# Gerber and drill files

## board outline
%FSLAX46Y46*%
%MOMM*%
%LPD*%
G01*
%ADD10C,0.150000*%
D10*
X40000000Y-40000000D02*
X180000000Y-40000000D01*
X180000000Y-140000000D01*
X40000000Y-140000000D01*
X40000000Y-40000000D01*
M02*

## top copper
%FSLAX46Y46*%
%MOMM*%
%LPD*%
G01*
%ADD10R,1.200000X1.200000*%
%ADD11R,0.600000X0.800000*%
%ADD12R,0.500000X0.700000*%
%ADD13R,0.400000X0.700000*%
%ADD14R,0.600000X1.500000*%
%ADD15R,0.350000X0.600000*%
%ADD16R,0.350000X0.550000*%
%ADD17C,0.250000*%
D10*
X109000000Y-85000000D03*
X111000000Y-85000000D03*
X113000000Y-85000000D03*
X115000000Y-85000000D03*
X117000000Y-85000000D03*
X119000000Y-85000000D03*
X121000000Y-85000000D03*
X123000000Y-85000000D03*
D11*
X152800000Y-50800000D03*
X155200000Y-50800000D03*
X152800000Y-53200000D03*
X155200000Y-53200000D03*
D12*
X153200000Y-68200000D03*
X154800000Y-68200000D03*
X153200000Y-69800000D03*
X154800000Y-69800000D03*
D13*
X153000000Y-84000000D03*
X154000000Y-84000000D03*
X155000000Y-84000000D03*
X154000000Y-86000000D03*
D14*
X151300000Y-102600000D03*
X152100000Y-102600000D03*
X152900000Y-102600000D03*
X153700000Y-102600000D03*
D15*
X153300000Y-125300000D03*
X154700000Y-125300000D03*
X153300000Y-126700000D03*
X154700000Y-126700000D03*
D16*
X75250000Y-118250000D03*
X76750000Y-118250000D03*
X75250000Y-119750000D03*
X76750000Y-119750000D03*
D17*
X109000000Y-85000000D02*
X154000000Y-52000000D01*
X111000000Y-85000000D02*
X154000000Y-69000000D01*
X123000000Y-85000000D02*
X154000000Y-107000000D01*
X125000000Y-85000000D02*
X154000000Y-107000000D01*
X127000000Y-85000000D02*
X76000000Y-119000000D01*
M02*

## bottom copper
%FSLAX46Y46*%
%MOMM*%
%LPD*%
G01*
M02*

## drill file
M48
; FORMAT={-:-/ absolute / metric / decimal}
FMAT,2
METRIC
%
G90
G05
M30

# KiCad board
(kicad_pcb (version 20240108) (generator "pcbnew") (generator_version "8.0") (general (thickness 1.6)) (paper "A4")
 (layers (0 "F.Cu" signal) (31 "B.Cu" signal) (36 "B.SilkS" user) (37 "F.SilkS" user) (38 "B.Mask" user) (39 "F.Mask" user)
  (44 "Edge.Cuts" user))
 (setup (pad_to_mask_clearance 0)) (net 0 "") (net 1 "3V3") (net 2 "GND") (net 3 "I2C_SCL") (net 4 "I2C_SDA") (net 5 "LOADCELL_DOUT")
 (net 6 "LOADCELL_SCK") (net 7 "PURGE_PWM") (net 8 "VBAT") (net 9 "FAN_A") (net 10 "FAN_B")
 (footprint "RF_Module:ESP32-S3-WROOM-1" (layer "F.Cu") (at 118 94) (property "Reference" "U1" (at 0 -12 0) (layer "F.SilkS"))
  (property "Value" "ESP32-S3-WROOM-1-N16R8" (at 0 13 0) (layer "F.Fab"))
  (pad "1" smd rect (at -9 -9) (size 1.2 1.2) (layers "F.Cu" "F.Mask") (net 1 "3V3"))
  (pad "2" smd rect (at -7 -9) (size 1.2 1.2) (layers "F.Cu" "F.Mask") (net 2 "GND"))
  (pad "3" smd rect (at -5 -9) (size 1.2 1.2) (layers "F.Cu" "F.Mask") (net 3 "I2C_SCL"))
  (pad "4" smd rect (at -3 -9) (size 1.2 1.2) (layers "F.Cu" "F.Mask") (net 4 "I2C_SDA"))
  (pad "5" smd rect (at -1 -9) (size 1.2 1.2) (layers "F.Cu" "F.Mask") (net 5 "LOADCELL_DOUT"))
  (pad "6" smd rect (at 1 -9) (size 1.2 1.2) (layers "F.Cu" "F.Mask") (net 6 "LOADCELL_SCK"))
  (pad "7" smd rect (at 3 -9) (size 1.2 1.2) (layers "F.Cu" "F.Mask") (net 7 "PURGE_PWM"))
  (pad "8" smd rect (at 5 -9) (size 1.2 1.2) (layers "F.Cu" "F.Mask") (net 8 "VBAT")))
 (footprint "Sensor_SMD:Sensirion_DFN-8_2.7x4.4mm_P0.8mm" (layer "F.Cu") (at 154 52)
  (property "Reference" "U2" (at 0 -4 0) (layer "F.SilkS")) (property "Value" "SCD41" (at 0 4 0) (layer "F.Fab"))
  (pad "1" smd rect (at -1.2 -1.2) (size 0.6 0.8) (layers "F.Cu" "F.Mask") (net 1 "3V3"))
  (pad "2" smd rect (at 1.2 -1.2) (size 0.6 0.8) (layers "F.Cu" "F.Mask") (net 3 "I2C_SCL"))
  (pad "3" smd rect (at -1.2 1.2) (size 0.6 0.8) (layers "F.Cu" "F.Mask") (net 4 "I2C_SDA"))
  (pad "4" smd rect (at 1.2 1.2) (size 0.6 0.8) (layers "F.Cu" "F.Mask") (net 2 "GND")))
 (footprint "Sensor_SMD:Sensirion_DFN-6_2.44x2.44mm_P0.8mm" (layer "F.Cu") (at 154 69)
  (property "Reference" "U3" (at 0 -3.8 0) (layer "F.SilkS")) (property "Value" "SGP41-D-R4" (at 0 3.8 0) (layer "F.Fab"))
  (pad "1" smd rect (at -0.8 -0.8) (size 0.5 0.7) (layers "F.Cu" "F.Mask") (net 1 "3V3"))
  (pad "2" smd rect (at 0.8 -0.8) (size 0.5 0.7) (layers "F.Cu" "F.Mask") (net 3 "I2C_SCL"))
  (pad "3" smd rect (at -0.8 0.8) (size 0.5 0.7) (layers "F.Cu" "F.Mask") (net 4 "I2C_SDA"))
  (pad "4" smd rect (at 0.8 0.8) (size 0.5 0.7) (layers "F.Cu" "F.Mask") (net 2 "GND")))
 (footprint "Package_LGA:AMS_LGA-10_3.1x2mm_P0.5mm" (layer "F.Cu") (at 154 85) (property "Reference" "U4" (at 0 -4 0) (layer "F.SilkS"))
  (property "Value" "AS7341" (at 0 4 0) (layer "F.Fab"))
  (pad "1" smd rect (at -1 -1) (size 0.4 0.7) (layers "F.Cu" "F.Mask") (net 1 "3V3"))
  (pad "2" smd rect (at 0 -1) (size 0.4 0.7) (layers "F.Cu" "F.Mask") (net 3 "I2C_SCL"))
  (pad "3" smd rect (at 1 -1) (size 0.4 0.7) (layers "F.Cu" "F.Mask") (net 4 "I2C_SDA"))
  (pad "4" smd rect (at 0 1) (size 0.4 0.7) (layers "F.Cu" "F.Mask") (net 2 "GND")))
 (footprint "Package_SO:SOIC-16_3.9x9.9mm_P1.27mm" (layer "F.Cu") (at 154 107) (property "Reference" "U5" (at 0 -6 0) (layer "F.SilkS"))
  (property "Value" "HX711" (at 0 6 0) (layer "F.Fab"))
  (pad "1" smd rect (at -2.7 -4.4) (size 0.6 1.5) (layers "F.Cu" "F.Mask") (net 1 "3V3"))
  (pad "2" smd rect (at -1.9 -4.4) (size 0.6 1.5) (layers "F.Cu" "F.Mask") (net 5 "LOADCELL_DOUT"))
  (pad "3" smd rect (at -1.1 -4.4) (size 0.6 1.5) (layers "F.Cu" "F.Mask") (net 6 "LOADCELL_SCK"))
  (pad "4" smd rect (at -0.3 -4.4) (size 0.6 1.5) (layers "F.Cu" "F.Mask") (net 2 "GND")))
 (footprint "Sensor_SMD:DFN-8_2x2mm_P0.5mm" (layer "F.Cu") (at 154 126) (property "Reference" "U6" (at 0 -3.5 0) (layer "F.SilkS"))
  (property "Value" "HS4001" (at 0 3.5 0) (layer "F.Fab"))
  (pad "1" smd rect (at -0.7 -0.7) (size 0.35 0.6) (layers "F.Cu" "F.Mask") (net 1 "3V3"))
  (pad "2" smd rect (at 0.7 -0.7) (size 0.35 0.6) (layers "F.Cu" "F.Mask") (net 3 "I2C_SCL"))
  (pad "3" smd rect (at -0.7 0.7) (size 0.35 0.6) (layers "F.Cu" "F.Mask") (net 4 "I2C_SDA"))
  (pad "4" smd rect (at 0.7 0.7) (size 0.35 0.6) (layers "F.Cu" "F.Mask") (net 2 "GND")))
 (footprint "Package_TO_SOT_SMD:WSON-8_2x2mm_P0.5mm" (layer "F.Cu") (at 76 119) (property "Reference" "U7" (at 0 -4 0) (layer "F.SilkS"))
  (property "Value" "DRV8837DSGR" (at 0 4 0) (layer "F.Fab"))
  (pad "1" smd rect (at -0.75 -0.75) (size 0.35 0.55) (layers "F.Cu" "F.Mask") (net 7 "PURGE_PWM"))
  (pad "2" smd rect (at 0.75 -0.75) (size 0.35 0.55) (layers "F.Cu" "F.Mask") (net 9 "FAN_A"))
  (pad "3" smd rect (at -0.75 0.75) (size 0.35 0.55) (layers "F.Cu" "F.Mask") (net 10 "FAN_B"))
  (pad "4" smd rect (at 0.75 0.75) (size 0.35 0.55) (layers "F.Cu" "F.Mask") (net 2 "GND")))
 (gr_rect (start 40 40) (end 180 140) (stroke (width 0.15) (type default)) (fill none) (layer "Edge.Cuts"))
 (segment (start 109 85) (end 154 52) (width 0.25) (layer "F.Cu") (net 3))
 (segment (start 111 85) (end 154 69) (width 0.25) (layer "F.Cu") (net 4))
 (segment (start 123 85) (end 154 107) (width 0.25) (layer "F.Cu") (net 5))
 (segment (start 125 85) (end 154 107) (width 0.25) (layer "F.Cu") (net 6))
 (segment (start 127 85) (end 76 119) (width 0.25) (layer "F.Cu") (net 7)))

